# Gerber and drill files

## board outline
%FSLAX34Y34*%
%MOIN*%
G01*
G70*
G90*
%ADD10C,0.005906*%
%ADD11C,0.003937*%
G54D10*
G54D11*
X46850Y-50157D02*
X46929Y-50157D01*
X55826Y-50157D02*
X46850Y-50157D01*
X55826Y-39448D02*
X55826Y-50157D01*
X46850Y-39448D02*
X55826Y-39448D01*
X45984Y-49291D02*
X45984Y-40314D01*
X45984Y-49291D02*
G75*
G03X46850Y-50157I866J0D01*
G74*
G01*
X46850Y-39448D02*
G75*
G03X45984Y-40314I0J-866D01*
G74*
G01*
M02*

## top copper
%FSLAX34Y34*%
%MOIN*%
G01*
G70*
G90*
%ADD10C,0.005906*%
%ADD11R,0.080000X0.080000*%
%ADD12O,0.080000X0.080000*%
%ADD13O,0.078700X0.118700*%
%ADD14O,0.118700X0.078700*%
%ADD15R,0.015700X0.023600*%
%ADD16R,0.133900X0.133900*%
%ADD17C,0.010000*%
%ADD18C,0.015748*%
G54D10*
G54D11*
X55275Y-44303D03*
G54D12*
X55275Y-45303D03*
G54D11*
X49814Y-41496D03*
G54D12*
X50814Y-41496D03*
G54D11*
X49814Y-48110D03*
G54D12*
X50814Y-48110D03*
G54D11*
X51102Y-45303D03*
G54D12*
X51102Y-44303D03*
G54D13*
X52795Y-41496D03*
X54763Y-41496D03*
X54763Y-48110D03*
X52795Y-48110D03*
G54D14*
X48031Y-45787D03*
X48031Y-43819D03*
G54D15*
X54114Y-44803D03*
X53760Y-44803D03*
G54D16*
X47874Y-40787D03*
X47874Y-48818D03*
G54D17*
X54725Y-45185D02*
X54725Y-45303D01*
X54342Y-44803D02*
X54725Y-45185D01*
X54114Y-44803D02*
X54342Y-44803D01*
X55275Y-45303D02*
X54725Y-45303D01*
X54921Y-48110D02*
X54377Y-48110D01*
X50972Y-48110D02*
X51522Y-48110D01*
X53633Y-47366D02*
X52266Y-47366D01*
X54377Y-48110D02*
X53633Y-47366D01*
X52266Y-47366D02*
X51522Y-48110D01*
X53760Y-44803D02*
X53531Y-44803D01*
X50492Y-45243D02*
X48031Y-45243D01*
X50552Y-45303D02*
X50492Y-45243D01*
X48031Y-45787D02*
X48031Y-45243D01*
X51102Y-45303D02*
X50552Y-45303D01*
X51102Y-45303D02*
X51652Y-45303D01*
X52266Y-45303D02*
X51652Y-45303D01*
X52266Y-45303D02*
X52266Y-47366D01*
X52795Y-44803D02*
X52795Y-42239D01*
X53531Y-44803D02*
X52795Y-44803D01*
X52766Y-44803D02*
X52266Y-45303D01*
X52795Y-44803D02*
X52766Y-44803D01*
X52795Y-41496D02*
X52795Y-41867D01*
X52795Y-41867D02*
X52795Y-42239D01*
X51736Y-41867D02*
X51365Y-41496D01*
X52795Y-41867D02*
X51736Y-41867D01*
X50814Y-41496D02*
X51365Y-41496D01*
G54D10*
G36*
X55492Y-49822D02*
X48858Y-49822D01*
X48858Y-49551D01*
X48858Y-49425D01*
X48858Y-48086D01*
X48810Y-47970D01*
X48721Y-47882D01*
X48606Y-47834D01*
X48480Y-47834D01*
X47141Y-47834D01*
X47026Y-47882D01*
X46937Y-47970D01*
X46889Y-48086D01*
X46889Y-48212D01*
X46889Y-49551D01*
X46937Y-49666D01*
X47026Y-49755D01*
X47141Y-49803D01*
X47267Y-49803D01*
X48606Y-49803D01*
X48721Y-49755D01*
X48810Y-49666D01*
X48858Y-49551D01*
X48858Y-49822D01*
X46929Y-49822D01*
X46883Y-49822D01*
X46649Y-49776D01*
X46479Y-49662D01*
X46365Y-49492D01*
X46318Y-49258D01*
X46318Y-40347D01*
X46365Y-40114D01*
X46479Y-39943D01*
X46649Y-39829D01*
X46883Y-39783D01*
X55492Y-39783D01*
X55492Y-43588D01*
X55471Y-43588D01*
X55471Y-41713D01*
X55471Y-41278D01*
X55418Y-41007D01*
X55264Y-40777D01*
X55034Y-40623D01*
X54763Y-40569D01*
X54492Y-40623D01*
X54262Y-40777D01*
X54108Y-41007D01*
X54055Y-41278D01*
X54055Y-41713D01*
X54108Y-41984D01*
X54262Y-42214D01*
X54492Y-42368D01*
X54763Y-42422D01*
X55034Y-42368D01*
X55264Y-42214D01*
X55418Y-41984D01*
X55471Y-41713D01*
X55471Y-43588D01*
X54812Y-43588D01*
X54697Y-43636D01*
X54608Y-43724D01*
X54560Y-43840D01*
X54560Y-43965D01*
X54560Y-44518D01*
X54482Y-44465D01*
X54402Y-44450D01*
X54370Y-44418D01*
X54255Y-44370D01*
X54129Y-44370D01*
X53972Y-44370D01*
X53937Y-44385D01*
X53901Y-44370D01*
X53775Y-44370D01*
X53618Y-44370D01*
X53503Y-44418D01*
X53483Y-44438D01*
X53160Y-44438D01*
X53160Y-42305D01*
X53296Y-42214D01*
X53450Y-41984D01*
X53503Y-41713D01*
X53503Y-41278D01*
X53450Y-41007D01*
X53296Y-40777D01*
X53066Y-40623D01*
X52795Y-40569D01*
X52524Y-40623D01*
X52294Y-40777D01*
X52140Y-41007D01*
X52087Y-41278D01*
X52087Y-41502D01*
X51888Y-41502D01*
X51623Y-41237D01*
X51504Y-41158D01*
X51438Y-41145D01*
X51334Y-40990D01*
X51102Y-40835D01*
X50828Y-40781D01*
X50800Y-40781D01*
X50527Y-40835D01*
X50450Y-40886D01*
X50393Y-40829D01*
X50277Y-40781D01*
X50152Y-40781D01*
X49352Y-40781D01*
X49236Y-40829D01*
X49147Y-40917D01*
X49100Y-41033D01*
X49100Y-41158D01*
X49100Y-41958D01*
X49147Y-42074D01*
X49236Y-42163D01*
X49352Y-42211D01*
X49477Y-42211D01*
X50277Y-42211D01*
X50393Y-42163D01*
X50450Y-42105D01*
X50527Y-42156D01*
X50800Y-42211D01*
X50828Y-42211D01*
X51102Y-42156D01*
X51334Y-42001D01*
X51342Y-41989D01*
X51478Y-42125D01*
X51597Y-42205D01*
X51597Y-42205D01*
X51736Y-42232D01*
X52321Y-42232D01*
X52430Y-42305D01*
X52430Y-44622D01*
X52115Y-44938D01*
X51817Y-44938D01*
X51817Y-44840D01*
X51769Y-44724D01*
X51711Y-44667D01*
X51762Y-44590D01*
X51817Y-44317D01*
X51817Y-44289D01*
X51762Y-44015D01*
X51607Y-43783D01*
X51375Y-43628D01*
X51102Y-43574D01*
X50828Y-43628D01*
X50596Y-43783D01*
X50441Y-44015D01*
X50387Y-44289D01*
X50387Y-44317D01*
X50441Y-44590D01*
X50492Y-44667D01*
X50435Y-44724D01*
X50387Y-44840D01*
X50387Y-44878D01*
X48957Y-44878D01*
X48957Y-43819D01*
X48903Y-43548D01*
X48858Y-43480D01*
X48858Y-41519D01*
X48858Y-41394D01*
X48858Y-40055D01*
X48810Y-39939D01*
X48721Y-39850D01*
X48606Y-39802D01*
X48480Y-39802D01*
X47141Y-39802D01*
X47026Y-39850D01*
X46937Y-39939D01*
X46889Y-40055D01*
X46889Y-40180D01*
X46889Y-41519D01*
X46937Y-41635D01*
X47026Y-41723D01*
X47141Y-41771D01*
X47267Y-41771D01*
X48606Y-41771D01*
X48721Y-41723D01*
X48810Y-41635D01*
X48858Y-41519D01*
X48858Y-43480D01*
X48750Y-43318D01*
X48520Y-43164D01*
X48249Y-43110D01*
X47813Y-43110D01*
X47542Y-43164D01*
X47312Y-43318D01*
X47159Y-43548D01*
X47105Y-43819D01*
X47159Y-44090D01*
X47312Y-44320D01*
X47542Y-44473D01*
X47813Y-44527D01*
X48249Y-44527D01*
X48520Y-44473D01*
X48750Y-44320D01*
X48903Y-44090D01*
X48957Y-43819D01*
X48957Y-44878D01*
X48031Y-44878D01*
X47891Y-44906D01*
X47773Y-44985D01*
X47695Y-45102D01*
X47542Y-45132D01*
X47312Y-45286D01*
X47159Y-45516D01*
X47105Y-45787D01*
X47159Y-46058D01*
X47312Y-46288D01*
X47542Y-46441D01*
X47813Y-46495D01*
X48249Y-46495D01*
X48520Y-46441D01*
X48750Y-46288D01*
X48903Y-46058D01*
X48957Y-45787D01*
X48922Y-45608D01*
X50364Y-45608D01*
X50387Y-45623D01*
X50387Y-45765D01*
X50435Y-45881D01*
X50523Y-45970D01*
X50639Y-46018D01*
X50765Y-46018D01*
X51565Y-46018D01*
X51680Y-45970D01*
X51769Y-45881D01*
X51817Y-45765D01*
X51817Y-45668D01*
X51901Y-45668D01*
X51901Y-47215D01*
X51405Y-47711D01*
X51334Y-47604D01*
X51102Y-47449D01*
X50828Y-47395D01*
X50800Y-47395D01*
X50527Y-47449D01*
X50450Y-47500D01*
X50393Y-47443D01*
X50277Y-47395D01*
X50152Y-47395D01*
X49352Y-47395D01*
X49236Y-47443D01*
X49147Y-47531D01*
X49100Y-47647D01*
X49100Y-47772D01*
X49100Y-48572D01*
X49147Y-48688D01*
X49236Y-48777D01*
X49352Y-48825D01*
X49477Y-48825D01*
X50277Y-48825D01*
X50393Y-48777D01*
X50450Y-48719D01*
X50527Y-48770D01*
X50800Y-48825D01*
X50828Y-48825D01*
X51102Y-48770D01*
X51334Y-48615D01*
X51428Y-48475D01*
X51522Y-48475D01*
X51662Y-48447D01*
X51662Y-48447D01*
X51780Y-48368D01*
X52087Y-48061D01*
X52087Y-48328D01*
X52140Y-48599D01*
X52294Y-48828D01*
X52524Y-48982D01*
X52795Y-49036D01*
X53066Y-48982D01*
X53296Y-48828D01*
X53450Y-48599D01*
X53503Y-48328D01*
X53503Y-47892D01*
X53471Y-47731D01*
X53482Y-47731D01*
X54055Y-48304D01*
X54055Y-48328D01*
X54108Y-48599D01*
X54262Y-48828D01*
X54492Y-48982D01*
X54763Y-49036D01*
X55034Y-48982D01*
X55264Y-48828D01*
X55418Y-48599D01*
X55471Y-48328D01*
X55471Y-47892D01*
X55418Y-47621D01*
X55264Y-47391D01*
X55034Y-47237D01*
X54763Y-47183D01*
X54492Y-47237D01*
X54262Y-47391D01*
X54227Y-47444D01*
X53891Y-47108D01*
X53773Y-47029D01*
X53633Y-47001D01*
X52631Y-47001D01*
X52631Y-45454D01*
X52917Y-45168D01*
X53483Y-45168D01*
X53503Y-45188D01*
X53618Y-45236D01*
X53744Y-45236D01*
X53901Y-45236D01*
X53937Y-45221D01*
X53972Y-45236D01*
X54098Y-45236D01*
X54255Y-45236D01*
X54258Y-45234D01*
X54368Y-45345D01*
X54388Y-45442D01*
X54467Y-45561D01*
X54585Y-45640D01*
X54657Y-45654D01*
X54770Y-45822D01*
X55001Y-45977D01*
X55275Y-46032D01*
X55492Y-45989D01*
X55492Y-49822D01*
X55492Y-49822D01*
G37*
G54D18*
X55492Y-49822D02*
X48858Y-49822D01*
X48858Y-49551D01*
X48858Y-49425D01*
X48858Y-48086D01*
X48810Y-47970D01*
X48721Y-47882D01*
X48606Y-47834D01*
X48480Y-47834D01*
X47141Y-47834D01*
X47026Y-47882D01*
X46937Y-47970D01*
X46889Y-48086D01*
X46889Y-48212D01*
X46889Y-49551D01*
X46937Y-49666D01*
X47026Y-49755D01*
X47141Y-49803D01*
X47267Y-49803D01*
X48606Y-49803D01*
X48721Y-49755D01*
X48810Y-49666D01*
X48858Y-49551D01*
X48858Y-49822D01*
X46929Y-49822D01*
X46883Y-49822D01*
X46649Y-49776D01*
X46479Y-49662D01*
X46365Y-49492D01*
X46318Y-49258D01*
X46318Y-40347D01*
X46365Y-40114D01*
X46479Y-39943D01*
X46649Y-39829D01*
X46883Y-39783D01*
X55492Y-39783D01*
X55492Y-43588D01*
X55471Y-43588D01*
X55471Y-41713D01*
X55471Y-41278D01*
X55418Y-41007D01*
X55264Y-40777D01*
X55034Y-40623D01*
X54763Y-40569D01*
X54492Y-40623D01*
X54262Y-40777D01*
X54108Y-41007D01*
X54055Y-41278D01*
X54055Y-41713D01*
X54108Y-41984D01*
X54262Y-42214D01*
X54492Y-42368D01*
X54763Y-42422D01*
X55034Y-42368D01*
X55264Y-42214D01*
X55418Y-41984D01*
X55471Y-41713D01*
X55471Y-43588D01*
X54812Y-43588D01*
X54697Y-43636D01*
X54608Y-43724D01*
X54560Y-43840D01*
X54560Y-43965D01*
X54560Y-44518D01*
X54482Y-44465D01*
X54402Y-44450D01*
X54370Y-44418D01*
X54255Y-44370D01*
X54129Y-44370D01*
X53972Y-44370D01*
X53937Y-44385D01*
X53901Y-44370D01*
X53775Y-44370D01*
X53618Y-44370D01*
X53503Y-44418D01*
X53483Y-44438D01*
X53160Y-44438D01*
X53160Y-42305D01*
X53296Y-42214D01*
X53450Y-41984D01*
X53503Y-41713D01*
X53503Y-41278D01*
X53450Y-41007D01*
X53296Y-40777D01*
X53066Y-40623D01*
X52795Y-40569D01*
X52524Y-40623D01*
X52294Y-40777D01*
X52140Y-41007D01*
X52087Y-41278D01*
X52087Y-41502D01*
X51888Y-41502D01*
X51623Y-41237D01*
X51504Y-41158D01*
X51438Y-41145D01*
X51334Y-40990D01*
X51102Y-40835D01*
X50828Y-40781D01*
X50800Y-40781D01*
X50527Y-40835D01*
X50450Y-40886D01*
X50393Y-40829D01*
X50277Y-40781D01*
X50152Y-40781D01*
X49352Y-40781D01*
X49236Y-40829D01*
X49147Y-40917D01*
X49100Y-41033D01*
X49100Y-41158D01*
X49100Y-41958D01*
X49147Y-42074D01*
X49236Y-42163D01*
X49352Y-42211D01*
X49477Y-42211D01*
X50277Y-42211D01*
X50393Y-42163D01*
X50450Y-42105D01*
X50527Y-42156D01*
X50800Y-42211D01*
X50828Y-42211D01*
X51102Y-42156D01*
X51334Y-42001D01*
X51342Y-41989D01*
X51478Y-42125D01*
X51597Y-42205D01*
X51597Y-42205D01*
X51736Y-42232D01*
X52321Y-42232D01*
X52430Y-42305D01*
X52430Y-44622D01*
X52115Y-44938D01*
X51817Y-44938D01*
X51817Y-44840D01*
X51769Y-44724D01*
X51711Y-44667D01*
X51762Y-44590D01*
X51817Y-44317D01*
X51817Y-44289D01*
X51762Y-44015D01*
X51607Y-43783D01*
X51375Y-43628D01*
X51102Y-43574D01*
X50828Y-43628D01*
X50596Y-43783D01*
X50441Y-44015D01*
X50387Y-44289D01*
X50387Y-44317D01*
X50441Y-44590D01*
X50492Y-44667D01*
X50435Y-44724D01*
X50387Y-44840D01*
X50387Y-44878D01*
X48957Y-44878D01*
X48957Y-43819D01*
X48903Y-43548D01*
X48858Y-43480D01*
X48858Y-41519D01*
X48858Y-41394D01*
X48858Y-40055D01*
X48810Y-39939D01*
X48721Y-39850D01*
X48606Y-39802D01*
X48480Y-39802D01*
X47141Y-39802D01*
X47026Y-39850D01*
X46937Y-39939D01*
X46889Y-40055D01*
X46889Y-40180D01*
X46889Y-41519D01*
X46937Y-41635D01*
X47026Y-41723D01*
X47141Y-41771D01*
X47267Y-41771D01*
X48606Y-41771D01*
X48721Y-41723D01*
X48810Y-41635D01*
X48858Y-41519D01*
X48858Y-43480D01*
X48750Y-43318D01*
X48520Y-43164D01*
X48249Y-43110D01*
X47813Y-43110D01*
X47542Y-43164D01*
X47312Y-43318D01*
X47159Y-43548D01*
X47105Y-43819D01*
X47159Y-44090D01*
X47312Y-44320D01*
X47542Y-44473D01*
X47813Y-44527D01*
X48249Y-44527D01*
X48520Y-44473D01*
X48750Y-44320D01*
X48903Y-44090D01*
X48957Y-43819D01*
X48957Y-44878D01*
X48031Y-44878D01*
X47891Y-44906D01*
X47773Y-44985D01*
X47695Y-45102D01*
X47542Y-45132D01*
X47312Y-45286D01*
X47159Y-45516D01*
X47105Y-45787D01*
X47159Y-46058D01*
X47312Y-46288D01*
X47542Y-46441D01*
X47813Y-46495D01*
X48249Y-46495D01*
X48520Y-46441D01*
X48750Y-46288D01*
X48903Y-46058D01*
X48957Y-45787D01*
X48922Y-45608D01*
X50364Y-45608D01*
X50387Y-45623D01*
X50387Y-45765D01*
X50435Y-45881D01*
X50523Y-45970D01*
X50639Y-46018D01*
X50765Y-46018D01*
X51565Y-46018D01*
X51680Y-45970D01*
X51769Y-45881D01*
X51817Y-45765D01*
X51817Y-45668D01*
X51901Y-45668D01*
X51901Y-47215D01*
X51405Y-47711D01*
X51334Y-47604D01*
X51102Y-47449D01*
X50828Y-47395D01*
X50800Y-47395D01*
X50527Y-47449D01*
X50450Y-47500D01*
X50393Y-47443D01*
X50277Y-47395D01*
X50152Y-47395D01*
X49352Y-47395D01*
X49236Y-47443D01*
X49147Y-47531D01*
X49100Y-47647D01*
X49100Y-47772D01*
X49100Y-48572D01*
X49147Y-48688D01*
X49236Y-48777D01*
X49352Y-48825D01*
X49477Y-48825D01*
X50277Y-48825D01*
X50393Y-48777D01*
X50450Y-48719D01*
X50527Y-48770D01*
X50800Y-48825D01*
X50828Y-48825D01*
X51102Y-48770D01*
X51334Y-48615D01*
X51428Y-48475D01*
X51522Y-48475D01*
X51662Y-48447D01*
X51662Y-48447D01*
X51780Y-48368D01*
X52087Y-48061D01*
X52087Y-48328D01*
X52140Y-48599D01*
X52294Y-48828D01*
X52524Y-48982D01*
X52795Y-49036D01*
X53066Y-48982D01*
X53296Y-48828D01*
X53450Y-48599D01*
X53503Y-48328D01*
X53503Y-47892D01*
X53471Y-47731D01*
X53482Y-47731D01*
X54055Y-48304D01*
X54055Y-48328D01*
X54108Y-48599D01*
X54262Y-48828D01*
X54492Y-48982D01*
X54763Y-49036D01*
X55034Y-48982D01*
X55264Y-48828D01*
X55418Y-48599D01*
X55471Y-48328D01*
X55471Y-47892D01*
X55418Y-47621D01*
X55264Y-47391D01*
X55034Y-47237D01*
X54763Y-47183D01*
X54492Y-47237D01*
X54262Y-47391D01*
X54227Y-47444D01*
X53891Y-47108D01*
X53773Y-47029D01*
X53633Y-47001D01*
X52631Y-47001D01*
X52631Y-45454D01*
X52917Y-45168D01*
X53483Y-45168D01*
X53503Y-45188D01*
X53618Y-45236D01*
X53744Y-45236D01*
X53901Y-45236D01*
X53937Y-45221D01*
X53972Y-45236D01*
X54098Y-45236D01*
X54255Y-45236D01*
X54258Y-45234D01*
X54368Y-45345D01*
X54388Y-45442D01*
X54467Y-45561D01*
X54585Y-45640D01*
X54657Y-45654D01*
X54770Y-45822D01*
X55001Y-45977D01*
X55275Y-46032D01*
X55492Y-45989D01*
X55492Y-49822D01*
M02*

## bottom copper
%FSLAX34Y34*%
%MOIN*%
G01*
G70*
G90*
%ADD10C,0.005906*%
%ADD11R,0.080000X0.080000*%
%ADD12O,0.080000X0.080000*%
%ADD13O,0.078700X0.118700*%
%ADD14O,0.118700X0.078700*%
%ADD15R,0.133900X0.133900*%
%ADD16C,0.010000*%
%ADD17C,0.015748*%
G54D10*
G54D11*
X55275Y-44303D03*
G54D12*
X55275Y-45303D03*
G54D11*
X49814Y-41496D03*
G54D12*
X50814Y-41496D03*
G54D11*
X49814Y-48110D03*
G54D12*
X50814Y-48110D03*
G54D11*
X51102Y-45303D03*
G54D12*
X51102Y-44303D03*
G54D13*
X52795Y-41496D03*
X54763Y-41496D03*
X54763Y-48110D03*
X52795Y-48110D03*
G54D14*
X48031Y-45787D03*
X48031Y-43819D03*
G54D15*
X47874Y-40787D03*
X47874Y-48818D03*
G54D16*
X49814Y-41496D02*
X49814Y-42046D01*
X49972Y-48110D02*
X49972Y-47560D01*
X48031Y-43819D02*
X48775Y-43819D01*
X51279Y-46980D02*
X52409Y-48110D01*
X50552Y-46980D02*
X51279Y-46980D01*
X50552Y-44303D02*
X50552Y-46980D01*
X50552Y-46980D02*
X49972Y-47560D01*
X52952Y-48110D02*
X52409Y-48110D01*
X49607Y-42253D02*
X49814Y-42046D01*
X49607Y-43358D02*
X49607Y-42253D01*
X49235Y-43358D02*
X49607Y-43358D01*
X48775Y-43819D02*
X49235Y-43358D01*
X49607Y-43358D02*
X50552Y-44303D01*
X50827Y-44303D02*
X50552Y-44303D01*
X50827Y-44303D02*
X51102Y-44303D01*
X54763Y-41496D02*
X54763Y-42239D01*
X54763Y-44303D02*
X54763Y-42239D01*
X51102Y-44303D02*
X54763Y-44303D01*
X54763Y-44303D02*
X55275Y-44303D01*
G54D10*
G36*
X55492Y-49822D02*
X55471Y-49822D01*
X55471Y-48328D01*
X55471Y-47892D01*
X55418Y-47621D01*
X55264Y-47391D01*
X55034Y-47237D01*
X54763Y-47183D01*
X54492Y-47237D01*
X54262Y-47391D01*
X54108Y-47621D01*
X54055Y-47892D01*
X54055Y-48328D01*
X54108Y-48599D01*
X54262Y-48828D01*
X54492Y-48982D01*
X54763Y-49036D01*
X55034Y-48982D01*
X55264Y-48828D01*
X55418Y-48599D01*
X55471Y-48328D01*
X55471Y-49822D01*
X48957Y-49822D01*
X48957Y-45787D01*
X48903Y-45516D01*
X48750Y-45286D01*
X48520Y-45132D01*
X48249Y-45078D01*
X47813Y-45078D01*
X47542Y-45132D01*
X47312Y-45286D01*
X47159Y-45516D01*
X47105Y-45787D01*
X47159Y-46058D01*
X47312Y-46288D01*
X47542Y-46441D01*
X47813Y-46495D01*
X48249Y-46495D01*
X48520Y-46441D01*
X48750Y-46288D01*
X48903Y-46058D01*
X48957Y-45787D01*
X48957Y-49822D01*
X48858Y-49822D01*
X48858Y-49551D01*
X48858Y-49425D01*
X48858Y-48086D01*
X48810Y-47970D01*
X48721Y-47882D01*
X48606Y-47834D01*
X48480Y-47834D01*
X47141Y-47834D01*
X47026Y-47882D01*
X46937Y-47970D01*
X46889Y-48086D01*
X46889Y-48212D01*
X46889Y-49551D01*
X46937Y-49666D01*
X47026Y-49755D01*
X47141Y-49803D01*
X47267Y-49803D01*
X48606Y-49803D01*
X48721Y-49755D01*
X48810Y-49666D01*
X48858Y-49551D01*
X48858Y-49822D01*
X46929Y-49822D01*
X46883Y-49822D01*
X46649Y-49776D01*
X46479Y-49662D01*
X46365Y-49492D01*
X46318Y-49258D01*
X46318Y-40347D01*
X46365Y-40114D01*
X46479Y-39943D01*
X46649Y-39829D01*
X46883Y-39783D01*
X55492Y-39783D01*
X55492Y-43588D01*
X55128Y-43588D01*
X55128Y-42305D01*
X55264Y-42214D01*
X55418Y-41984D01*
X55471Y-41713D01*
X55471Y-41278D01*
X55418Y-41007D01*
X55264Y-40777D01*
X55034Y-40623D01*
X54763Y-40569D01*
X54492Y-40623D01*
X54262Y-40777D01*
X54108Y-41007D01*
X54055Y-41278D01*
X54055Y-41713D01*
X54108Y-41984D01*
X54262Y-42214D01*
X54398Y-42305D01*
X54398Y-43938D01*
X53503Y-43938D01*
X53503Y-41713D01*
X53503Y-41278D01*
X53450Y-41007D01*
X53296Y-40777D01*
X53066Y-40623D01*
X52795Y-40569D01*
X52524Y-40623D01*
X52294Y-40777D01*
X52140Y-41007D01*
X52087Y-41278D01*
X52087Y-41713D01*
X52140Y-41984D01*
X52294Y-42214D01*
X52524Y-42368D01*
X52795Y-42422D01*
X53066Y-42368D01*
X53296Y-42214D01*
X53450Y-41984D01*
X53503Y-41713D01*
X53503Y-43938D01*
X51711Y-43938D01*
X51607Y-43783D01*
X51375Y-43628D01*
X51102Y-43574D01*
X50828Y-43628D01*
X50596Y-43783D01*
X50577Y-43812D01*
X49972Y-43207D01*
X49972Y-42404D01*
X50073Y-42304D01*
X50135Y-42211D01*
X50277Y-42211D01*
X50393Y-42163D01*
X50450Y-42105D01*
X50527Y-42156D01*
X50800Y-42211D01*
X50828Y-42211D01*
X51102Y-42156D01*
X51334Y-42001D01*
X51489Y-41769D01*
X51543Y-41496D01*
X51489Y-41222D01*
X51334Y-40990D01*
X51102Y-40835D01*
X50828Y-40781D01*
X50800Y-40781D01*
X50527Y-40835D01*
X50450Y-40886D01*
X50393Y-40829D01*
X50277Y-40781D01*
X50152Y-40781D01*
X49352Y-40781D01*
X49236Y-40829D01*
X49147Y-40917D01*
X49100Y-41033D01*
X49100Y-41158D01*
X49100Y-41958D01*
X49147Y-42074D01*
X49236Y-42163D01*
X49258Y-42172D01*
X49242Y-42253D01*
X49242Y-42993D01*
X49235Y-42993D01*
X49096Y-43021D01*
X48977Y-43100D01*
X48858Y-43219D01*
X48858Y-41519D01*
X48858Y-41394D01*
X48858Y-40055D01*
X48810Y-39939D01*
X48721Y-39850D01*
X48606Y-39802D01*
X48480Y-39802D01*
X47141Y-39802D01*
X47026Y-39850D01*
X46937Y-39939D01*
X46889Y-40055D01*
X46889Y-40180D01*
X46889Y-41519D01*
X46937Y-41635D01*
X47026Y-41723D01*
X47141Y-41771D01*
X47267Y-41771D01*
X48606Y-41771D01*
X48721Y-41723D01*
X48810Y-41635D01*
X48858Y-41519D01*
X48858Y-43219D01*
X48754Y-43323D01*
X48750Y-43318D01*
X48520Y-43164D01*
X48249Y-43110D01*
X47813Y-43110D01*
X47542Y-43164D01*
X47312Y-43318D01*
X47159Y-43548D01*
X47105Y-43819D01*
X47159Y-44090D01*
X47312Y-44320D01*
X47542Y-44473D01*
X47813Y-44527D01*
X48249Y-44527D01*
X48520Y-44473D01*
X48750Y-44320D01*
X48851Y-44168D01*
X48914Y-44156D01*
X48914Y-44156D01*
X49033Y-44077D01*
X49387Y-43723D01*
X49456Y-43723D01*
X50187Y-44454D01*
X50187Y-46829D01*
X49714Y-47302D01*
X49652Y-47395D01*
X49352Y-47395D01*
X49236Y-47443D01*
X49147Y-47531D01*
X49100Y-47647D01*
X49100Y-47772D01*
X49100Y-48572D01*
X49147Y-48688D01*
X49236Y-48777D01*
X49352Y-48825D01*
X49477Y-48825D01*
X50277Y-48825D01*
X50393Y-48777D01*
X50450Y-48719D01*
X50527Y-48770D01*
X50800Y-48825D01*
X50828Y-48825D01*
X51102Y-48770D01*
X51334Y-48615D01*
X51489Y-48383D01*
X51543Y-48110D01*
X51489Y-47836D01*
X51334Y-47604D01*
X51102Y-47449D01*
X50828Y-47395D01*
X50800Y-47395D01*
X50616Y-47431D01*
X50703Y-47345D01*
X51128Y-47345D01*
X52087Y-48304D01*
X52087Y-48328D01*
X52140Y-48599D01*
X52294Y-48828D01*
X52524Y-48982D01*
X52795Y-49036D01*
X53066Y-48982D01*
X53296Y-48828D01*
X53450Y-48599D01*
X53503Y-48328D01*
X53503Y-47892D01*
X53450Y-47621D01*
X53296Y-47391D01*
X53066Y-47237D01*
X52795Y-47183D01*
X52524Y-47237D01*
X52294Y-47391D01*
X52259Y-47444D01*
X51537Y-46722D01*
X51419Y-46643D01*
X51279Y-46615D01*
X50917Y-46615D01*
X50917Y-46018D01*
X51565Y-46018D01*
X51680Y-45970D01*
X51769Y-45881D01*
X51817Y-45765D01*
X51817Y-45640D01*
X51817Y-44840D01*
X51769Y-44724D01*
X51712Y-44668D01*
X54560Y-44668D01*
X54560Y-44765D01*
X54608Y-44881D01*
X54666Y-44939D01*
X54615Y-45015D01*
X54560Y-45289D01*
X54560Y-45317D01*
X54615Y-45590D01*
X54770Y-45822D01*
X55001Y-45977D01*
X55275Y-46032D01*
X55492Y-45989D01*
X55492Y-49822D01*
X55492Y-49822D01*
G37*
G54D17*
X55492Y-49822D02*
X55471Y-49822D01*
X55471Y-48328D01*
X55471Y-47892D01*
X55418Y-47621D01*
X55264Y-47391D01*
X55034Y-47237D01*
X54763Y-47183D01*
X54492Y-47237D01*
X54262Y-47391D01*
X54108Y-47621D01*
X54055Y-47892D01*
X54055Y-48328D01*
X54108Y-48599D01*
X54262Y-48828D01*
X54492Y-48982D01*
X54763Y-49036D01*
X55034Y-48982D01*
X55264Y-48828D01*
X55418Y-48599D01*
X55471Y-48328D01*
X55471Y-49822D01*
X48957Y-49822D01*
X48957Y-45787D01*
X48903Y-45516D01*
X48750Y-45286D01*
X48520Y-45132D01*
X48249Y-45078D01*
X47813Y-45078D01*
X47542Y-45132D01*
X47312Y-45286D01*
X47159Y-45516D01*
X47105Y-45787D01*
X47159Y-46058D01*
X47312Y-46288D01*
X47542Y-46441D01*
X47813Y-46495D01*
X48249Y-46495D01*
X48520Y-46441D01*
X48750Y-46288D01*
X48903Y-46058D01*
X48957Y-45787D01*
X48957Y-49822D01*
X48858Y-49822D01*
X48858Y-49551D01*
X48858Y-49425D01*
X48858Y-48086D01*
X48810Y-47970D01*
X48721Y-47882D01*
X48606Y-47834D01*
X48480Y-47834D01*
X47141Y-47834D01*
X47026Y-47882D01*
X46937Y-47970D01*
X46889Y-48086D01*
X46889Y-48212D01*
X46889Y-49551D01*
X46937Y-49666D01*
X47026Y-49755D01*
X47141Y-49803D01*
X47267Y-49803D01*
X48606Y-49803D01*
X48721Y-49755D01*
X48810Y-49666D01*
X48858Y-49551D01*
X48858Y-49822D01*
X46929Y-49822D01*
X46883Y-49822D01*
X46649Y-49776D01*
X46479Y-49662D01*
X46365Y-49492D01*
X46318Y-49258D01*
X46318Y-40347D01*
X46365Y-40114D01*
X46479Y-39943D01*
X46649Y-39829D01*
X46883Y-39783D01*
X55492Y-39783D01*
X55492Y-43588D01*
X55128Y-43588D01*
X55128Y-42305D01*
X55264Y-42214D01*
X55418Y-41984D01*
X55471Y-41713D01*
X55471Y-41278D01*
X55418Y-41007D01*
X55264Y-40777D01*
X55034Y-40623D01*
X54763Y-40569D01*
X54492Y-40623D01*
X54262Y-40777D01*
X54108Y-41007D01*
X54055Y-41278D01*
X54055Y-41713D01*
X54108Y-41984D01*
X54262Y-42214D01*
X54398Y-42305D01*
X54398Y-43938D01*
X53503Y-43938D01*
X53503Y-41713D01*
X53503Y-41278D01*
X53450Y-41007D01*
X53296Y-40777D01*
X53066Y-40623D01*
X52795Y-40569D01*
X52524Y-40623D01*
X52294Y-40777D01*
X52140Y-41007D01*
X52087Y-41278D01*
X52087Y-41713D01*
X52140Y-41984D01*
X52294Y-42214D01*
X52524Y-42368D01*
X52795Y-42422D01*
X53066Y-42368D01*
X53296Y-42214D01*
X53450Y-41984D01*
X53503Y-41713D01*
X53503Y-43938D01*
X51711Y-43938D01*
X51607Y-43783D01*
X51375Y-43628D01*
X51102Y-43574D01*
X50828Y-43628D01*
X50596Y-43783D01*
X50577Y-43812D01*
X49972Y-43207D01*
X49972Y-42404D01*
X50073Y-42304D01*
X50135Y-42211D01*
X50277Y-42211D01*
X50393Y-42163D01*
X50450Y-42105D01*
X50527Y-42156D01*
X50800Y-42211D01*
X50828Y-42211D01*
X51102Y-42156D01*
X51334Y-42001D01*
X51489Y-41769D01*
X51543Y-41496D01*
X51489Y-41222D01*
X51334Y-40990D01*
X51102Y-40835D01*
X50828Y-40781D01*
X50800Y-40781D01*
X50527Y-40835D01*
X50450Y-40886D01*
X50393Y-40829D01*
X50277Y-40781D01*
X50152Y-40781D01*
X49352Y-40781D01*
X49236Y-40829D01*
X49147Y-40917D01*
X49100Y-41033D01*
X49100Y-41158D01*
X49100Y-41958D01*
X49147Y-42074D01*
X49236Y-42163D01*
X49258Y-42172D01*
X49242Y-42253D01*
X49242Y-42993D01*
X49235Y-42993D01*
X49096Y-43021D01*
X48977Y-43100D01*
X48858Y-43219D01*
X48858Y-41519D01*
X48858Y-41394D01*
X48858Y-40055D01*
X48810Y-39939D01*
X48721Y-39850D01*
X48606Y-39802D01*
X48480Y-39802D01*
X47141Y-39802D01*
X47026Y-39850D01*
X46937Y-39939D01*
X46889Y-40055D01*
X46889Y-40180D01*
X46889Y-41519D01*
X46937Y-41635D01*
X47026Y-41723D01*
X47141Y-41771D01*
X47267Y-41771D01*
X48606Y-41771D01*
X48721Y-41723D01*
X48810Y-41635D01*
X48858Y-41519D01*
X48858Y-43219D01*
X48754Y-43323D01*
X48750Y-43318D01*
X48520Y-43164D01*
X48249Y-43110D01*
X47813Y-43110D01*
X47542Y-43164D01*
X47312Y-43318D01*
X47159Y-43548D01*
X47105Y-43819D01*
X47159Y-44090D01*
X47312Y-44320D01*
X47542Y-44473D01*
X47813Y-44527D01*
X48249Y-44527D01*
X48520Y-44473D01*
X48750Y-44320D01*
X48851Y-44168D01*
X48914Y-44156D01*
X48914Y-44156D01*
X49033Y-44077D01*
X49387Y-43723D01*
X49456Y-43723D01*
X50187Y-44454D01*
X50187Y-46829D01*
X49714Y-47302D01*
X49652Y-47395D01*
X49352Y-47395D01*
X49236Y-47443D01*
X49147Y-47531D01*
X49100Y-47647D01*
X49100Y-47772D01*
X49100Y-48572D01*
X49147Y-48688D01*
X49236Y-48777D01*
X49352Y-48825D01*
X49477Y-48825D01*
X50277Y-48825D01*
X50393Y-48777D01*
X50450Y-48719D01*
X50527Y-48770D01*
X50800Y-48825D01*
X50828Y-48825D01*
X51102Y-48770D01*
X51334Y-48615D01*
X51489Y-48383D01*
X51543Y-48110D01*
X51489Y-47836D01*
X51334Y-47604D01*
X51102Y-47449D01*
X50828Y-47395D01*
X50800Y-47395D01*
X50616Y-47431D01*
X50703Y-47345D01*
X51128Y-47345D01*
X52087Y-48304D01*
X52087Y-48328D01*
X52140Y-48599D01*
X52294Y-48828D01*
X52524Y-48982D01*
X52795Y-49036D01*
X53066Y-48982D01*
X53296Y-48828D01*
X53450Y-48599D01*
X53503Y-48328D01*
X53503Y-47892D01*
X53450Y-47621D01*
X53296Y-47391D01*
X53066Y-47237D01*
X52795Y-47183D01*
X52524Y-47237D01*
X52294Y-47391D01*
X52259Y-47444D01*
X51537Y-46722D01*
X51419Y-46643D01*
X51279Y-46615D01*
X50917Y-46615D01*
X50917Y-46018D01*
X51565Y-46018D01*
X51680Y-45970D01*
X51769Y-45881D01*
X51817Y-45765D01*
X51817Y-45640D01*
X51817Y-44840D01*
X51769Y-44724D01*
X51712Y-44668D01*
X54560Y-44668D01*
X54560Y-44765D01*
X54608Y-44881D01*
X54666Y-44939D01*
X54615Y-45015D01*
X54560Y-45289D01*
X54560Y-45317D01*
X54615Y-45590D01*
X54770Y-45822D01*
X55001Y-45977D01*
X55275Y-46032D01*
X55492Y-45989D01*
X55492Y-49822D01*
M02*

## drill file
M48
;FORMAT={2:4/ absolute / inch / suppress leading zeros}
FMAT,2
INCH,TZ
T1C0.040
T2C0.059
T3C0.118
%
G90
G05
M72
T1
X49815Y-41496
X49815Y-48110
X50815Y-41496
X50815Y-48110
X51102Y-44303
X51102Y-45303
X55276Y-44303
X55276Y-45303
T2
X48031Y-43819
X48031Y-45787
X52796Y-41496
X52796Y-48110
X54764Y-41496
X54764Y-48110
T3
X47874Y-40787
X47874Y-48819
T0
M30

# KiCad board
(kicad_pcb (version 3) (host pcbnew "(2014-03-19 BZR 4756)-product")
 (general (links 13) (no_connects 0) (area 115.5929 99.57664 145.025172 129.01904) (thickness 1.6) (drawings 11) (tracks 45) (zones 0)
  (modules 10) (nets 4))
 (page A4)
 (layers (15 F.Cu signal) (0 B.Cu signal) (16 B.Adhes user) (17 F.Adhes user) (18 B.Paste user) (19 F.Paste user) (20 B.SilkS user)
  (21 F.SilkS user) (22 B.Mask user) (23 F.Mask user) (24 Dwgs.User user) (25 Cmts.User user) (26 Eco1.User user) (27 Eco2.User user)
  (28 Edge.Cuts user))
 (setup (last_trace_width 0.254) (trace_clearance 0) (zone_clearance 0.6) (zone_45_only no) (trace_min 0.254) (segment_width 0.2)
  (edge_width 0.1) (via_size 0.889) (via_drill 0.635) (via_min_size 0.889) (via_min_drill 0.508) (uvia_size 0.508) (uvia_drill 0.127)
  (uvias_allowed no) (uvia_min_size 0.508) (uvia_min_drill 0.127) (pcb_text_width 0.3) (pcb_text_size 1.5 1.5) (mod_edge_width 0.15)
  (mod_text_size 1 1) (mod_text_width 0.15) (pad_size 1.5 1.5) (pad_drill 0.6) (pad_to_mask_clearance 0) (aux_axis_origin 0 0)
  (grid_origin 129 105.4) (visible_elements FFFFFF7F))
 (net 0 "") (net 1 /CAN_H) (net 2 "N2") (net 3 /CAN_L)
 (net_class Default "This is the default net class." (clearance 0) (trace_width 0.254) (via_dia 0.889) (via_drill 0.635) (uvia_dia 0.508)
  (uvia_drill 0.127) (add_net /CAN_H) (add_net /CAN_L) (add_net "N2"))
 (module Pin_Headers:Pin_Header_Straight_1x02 (layer F.Cu) (at 140.4 113.8 270)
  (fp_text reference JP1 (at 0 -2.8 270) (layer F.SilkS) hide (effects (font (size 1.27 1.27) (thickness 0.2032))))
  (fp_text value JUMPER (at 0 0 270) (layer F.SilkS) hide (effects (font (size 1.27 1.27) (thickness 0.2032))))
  (pad 1 thru_hole rect (at -1.27 0 270) (size 2.032 2.032) (drill 1.016) (layers *.Cu *.Mask F.SilkS) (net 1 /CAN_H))
  (pad 2 thru_hole oval (at 1.27 0 270) (size 2.032 2.032) (drill 1.016) (layers *.Cu *.Mask F.SilkS) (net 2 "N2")))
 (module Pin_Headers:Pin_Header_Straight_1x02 (layer F.Cu) (at 127.8 105.4)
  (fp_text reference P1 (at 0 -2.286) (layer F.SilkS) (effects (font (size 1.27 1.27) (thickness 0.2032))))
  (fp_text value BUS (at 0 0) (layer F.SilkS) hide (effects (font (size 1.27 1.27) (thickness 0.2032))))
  (pad 1 thru_hole rect (at -1.27 0) (size 2.032 2.032) (drill 1.016) (layers *.Cu *.Mask F.SilkS) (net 1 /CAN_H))
  (pad 2 thru_hole oval (at 1.27 0) (size 2.032 2.032) (drill 1.016) (layers *.Cu *.Mask F.SilkS) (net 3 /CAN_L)))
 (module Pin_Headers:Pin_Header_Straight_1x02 (layer F.Cu) (at 127.8 122.2)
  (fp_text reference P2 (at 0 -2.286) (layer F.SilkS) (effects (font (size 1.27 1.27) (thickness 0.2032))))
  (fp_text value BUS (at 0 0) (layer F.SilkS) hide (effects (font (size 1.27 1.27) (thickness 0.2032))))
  (pad 1 thru_hole rect (at -1.27 0) (size 2.032 2.032) (drill 1.016) (layers *.Cu *.Mask F.SilkS) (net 1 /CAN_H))
  (pad 2 thru_hole oval (at 1.27 0) (size 2.032 2.032) (drill 1.016) (layers *.Cu *.Mask F.SilkS) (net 3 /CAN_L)))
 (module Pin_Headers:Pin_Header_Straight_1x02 (layer F.Cu) (at 129.8 113.8 90)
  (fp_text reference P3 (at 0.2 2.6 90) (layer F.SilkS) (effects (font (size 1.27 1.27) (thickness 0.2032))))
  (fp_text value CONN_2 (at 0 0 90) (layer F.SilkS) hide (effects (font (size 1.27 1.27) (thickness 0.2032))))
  (pad 1 thru_hole rect (at -1.27 0 90) (size 2.032 2.032) (drill 1.016) (layers *.Cu *.Mask F.SilkS) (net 3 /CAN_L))
  (pad 2 thru_hole oval (at 1.27 0 90) (size 2.032 2.032) (drill 1.016) (layers *.Cu *.Mask F.SilkS) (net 1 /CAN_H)))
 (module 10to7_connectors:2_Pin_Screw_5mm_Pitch (layer F.Cu) (at 136.6 105.4)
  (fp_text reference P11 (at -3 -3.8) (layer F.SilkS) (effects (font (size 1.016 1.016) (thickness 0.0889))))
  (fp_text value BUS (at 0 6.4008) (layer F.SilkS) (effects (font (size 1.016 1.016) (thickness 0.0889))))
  (pad 1 thru_hole oval (at -2.49936 0) (size 1.99898 3.01498) (drill 1.50114) (layers *.Cu F.Paste F.SilkS B.Mask) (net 3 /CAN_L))
  (pad 2 thru_hole oval (at 2.49936 0) (size 1.99898 3.01498) (drill 1.50114) (layers *.Cu F.Paste F.SilkS B.Mask) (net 1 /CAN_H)))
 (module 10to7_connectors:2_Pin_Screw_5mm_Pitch (layer F.Cu) (at 136.6 122.2 180)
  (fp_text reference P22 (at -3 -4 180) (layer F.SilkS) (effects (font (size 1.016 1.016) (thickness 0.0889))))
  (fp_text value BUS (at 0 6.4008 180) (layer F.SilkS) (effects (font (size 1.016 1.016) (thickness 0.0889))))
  (pad 1 thru_hole oval (at -2.49936 0 180) (size 1.99898 3.01498) (drill 1.50114) (layers *.Cu F.Paste F.SilkS B.Mask) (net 3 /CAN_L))
  (pad 2 thru_hole oval (at 2.49936 0 180) (size 1.99898 3.01498) (drill 1.50114) (layers *.Cu F.Paste F.SilkS B.Mask) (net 1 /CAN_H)))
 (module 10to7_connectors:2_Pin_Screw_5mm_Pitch (layer F.Cu) (at 122 113.8 90)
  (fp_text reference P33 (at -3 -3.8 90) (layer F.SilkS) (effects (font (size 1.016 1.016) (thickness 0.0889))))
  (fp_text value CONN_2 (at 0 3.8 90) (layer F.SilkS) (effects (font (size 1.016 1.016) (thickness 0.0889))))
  (pad 1 thru_hole oval (at -2.49936 0 90) (size 1.99898 3.01498) (drill 1.50114) (layers *.Cu F.Paste F.SilkS B.Mask) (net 3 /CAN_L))
  (pad 2 thru_hole oval (at 2.49936 0 90) (size 1.99898 3.01498) (drill 1.50114) (layers *.Cu F.Paste F.SilkS B.Mask) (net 1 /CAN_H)))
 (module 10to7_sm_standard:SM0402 (layer F.Cu) (at 137 113.8 180)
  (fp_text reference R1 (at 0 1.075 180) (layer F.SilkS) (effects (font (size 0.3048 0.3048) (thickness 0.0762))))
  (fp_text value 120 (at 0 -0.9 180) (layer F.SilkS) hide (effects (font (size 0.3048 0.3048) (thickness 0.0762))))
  (pad 1 smd rect (at -0.44958 0 180) (size 0.39878 0.59944) (layers F.Cu F.Paste F.Mask) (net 2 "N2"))
  (pad 2 smd rect (at 0.44958 0 180) (size 0.39878 0.59944) (layers F.Cu F.Paste F.Mask) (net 3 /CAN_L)))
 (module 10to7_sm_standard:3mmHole (layer F.Cu) (at 121.6 103.6)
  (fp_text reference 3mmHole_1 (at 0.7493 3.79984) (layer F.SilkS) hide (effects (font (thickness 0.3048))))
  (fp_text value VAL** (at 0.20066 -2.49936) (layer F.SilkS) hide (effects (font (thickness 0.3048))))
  (pad 1 thru_hole rect (at 0 0) (size 3.40106 3.40106) (drill 2.99974) (layers *.Cu *.Mask F.SilkS)))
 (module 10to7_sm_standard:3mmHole (layer F.Cu) (at 121.6 124)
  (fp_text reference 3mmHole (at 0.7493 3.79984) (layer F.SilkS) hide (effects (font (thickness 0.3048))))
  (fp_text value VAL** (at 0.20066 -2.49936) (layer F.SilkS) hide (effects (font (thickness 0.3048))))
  (pad 1 thru_hole rect (at 0 0) (size 3.40106 3.40106) (drill 2.99974) (layers *.Cu *.Mask F.SilkS)))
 (gr_line (start 119 127.4) (end 119.2 127.4) (angle 90) (layer Edge.Cuts) (width 0.1))
 (gr_line (start 141.8 127.4) (end 119 127.4) (angle 90) (layer Edge.Cuts) (width 0.1))
 (gr_line (start 141.8 100.2) (end 141.8 127.4) (angle 90) (layer Edge.Cuts) (width 0.1))
 (gr_line (start 119 100.2) (end 141.8 100.2) (angle 90) (layer Edge.Cuts) (width 0.1))
 (gr_line (start 116.8 125.2) (end 116.8 102.4) (angle 90) (layer Edge.Cuts) (width 0.1))
 (gr_arc (start 119 125.2) (end 119 127.4) (angle 90) (layer Edge.Cuts) (width 0.1))
 (gr_arc (start 119 102.4) (end 116.8 102.4) (angle 90) (layer Edge.Cuts) (width 0.1))
 (segment (start 126.53 105.4) (end 126.53 106.7973) (width 0.254) (layer B.Cu) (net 1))
 (segment (start 126.93 122.2) (end 126.93 120.8027) (width 0.254) (layer B.Cu) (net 1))
 (segment (start 122 111.3006) (end 123.8888 111.3006) (width 0.254) (layer B.Cu) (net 1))
 (segment (start 130.2498 119.33) (end 133.1198 122.2) (width 0.254) (layer B.Cu) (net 1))
 (segment (start 128.4027 119.33) (end 130.2498 119.33) (width 0.254) (layer B.Cu) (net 1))
 (segment (start 128.4027 112.53) (end 128.4027 119.33) (width 0.254) (layer B.Cu) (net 1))
 (segment (start 128.4027 119.33) (end 126.93 120.8027) (width 0.254) (layer B.Cu) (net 1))
 (segment (start 134.5006 122.2) (end 133.1198 122.2) (width 0.254) (layer B.Cu) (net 1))
 (segment (start 126.0028 107.3245) (end 126.53 106.7973) (width 0.254) (layer B.Cu) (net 1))
 (segment (start 126.0028 110.1301) (end 126.0028 107.3245) (width 0.254) (layer B.Cu) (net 1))
 (segment (start 125.0593 110.1301) (end 126.0028 110.1301) (width 0.254) (layer B.Cu) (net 1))
 (segment (start 123.8888 111.3006) (end 125.0593 110.1301) (width 0.254) (layer B.Cu) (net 1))
 (segment (start 126.0028 110.1301) (end 128.4027 112.53) (width 0.254) (layer B.Cu) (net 1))
 (segment (start 129.1014 112.53) (end 128.4027 112.53) (width 0.254) (layer B.Cu) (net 1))
 (segment (start 129.1014 112.53) (end 129.8 112.53) (width 0.254) (layer B.Cu) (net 1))
 (segment (start 139.0994 105.4) (end 139.0994 107.2888) (width 0.254) (layer B.Cu) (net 1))
 (segment (start 139.0994 112.53) (end 139.0994 107.2888) (width 0.254) (layer B.Cu) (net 1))
 (segment (start 129.8 112.53) (end 139.0994 112.53) (width 0.254) (layer B.Cu) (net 1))
 (segment (start 139.0994 112.53) (end 140.4 112.53) (width 0.254) (layer B.Cu) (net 1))
 (segment (start 139.0027 114.7724) (end 139.0027 115.07) (width 0.254) (layer F.Cu) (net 2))
 (segment (start 138.0303 113.8) (end 139.0027 114.7724) (width 0.254) (layer F.Cu) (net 2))
 (segment (start 137.4496 113.8) (end 138.0303 113.8) (width 0.254) (layer F.Cu) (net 2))
 (segment (start 140.4 115.07) (end 139.0027 115.07) (width 0.254) (layer F.Cu) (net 2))
 (segment (start 139.4994 122.2) (end 138.1186 122.2) (width 0.254) (layer F.Cu) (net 3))
 (segment (start 129.47 122.2) (end 130.8673 122.2) (width 0.254) (layer F.Cu) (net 3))
 (segment (start 136.2297 120.3111) (end 132.7562 120.3111) (width 0.254) (layer F.Cu) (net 3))
 (segment (start 138.1186 122.2) (end 136.2297 120.3111) (width 0.254) (layer F.Cu) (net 3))
 (segment (start 132.7562 120.3111) (end 130.8673 122.2) (width 0.254) (layer F.Cu) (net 3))
 (segment (start 136.5504 113.8) (end 135.9697 113.8) (width 0.254) (layer F.Cu) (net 3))
 (segment (start 128.2513 114.9186) (end 122 114.9186) (width 0.254) (layer F.Cu) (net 3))
 (segment (start 128.4027 115.07) (end 128.2513 114.9186) (width 0.254) (layer F.Cu) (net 3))
 (segment (start 122 116.2994) (end 122 114.9186) (width 0.254) (layer F.Cu) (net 3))
 (segment (start 129.8 115.07) (end 128.4027 115.07) (width 0.254) (layer F.Cu) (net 3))
 (segment (start 129.8 115.07) (end 131.1973 115.07) (width 0.254) (layer F.Cu) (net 3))
 (segment (start 132.7562 115.07) (end 131.1973 115.07) (width 0.254) (layer F.Cu) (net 3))
 (segment (start 132.7562 115.07) (end 132.7562 120.3111) (width 0.254) (layer F.Cu) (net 3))
 (segment (start 134.1006 113.8) (end 134.1006 107.2888) (width 0.254) (layer F.Cu) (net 3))
 (segment (start 135.9697 113.8) (end 134.1006 113.8) (width 0.254) (layer F.Cu) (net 3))
 (segment (start 134.0262 113.8) (end 132.7562 115.07) (width 0.254) (layer F.Cu) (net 3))
 (segment (start 134.1006 113.8) (end 134.0262 113.8) (width 0.254) (layer F.Cu) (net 3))
 (segment (start 134.1006 105.4) (end 134.1006 106.3444) (width 0.254) (layer F.Cu) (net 3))
 (segment (start 134.1006 106.3444) (end 134.1006 107.2888) (width 0.254) (layer F.Cu) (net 3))
 (segment (start 131.4117 106.3444) (end 130.4673 105.4) (width 0.254) (layer F.Cu) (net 3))
 (segment (start 134.1006 106.3444) (end 131.4117 106.3444) (width 0.254) (layer F.Cu) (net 3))
 (segment (start 129.07 105.4) (end 130.4673 105.4) (width 0.254) (layer F.Cu) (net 3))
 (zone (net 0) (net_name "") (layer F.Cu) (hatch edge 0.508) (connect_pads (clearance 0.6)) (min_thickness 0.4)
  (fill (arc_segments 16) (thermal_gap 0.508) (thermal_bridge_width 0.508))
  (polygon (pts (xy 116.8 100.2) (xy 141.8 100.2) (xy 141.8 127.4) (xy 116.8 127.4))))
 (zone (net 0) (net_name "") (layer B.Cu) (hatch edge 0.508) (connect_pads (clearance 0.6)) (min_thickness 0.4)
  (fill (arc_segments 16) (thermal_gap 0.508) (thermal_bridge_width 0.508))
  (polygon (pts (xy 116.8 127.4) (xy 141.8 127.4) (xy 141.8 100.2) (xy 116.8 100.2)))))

